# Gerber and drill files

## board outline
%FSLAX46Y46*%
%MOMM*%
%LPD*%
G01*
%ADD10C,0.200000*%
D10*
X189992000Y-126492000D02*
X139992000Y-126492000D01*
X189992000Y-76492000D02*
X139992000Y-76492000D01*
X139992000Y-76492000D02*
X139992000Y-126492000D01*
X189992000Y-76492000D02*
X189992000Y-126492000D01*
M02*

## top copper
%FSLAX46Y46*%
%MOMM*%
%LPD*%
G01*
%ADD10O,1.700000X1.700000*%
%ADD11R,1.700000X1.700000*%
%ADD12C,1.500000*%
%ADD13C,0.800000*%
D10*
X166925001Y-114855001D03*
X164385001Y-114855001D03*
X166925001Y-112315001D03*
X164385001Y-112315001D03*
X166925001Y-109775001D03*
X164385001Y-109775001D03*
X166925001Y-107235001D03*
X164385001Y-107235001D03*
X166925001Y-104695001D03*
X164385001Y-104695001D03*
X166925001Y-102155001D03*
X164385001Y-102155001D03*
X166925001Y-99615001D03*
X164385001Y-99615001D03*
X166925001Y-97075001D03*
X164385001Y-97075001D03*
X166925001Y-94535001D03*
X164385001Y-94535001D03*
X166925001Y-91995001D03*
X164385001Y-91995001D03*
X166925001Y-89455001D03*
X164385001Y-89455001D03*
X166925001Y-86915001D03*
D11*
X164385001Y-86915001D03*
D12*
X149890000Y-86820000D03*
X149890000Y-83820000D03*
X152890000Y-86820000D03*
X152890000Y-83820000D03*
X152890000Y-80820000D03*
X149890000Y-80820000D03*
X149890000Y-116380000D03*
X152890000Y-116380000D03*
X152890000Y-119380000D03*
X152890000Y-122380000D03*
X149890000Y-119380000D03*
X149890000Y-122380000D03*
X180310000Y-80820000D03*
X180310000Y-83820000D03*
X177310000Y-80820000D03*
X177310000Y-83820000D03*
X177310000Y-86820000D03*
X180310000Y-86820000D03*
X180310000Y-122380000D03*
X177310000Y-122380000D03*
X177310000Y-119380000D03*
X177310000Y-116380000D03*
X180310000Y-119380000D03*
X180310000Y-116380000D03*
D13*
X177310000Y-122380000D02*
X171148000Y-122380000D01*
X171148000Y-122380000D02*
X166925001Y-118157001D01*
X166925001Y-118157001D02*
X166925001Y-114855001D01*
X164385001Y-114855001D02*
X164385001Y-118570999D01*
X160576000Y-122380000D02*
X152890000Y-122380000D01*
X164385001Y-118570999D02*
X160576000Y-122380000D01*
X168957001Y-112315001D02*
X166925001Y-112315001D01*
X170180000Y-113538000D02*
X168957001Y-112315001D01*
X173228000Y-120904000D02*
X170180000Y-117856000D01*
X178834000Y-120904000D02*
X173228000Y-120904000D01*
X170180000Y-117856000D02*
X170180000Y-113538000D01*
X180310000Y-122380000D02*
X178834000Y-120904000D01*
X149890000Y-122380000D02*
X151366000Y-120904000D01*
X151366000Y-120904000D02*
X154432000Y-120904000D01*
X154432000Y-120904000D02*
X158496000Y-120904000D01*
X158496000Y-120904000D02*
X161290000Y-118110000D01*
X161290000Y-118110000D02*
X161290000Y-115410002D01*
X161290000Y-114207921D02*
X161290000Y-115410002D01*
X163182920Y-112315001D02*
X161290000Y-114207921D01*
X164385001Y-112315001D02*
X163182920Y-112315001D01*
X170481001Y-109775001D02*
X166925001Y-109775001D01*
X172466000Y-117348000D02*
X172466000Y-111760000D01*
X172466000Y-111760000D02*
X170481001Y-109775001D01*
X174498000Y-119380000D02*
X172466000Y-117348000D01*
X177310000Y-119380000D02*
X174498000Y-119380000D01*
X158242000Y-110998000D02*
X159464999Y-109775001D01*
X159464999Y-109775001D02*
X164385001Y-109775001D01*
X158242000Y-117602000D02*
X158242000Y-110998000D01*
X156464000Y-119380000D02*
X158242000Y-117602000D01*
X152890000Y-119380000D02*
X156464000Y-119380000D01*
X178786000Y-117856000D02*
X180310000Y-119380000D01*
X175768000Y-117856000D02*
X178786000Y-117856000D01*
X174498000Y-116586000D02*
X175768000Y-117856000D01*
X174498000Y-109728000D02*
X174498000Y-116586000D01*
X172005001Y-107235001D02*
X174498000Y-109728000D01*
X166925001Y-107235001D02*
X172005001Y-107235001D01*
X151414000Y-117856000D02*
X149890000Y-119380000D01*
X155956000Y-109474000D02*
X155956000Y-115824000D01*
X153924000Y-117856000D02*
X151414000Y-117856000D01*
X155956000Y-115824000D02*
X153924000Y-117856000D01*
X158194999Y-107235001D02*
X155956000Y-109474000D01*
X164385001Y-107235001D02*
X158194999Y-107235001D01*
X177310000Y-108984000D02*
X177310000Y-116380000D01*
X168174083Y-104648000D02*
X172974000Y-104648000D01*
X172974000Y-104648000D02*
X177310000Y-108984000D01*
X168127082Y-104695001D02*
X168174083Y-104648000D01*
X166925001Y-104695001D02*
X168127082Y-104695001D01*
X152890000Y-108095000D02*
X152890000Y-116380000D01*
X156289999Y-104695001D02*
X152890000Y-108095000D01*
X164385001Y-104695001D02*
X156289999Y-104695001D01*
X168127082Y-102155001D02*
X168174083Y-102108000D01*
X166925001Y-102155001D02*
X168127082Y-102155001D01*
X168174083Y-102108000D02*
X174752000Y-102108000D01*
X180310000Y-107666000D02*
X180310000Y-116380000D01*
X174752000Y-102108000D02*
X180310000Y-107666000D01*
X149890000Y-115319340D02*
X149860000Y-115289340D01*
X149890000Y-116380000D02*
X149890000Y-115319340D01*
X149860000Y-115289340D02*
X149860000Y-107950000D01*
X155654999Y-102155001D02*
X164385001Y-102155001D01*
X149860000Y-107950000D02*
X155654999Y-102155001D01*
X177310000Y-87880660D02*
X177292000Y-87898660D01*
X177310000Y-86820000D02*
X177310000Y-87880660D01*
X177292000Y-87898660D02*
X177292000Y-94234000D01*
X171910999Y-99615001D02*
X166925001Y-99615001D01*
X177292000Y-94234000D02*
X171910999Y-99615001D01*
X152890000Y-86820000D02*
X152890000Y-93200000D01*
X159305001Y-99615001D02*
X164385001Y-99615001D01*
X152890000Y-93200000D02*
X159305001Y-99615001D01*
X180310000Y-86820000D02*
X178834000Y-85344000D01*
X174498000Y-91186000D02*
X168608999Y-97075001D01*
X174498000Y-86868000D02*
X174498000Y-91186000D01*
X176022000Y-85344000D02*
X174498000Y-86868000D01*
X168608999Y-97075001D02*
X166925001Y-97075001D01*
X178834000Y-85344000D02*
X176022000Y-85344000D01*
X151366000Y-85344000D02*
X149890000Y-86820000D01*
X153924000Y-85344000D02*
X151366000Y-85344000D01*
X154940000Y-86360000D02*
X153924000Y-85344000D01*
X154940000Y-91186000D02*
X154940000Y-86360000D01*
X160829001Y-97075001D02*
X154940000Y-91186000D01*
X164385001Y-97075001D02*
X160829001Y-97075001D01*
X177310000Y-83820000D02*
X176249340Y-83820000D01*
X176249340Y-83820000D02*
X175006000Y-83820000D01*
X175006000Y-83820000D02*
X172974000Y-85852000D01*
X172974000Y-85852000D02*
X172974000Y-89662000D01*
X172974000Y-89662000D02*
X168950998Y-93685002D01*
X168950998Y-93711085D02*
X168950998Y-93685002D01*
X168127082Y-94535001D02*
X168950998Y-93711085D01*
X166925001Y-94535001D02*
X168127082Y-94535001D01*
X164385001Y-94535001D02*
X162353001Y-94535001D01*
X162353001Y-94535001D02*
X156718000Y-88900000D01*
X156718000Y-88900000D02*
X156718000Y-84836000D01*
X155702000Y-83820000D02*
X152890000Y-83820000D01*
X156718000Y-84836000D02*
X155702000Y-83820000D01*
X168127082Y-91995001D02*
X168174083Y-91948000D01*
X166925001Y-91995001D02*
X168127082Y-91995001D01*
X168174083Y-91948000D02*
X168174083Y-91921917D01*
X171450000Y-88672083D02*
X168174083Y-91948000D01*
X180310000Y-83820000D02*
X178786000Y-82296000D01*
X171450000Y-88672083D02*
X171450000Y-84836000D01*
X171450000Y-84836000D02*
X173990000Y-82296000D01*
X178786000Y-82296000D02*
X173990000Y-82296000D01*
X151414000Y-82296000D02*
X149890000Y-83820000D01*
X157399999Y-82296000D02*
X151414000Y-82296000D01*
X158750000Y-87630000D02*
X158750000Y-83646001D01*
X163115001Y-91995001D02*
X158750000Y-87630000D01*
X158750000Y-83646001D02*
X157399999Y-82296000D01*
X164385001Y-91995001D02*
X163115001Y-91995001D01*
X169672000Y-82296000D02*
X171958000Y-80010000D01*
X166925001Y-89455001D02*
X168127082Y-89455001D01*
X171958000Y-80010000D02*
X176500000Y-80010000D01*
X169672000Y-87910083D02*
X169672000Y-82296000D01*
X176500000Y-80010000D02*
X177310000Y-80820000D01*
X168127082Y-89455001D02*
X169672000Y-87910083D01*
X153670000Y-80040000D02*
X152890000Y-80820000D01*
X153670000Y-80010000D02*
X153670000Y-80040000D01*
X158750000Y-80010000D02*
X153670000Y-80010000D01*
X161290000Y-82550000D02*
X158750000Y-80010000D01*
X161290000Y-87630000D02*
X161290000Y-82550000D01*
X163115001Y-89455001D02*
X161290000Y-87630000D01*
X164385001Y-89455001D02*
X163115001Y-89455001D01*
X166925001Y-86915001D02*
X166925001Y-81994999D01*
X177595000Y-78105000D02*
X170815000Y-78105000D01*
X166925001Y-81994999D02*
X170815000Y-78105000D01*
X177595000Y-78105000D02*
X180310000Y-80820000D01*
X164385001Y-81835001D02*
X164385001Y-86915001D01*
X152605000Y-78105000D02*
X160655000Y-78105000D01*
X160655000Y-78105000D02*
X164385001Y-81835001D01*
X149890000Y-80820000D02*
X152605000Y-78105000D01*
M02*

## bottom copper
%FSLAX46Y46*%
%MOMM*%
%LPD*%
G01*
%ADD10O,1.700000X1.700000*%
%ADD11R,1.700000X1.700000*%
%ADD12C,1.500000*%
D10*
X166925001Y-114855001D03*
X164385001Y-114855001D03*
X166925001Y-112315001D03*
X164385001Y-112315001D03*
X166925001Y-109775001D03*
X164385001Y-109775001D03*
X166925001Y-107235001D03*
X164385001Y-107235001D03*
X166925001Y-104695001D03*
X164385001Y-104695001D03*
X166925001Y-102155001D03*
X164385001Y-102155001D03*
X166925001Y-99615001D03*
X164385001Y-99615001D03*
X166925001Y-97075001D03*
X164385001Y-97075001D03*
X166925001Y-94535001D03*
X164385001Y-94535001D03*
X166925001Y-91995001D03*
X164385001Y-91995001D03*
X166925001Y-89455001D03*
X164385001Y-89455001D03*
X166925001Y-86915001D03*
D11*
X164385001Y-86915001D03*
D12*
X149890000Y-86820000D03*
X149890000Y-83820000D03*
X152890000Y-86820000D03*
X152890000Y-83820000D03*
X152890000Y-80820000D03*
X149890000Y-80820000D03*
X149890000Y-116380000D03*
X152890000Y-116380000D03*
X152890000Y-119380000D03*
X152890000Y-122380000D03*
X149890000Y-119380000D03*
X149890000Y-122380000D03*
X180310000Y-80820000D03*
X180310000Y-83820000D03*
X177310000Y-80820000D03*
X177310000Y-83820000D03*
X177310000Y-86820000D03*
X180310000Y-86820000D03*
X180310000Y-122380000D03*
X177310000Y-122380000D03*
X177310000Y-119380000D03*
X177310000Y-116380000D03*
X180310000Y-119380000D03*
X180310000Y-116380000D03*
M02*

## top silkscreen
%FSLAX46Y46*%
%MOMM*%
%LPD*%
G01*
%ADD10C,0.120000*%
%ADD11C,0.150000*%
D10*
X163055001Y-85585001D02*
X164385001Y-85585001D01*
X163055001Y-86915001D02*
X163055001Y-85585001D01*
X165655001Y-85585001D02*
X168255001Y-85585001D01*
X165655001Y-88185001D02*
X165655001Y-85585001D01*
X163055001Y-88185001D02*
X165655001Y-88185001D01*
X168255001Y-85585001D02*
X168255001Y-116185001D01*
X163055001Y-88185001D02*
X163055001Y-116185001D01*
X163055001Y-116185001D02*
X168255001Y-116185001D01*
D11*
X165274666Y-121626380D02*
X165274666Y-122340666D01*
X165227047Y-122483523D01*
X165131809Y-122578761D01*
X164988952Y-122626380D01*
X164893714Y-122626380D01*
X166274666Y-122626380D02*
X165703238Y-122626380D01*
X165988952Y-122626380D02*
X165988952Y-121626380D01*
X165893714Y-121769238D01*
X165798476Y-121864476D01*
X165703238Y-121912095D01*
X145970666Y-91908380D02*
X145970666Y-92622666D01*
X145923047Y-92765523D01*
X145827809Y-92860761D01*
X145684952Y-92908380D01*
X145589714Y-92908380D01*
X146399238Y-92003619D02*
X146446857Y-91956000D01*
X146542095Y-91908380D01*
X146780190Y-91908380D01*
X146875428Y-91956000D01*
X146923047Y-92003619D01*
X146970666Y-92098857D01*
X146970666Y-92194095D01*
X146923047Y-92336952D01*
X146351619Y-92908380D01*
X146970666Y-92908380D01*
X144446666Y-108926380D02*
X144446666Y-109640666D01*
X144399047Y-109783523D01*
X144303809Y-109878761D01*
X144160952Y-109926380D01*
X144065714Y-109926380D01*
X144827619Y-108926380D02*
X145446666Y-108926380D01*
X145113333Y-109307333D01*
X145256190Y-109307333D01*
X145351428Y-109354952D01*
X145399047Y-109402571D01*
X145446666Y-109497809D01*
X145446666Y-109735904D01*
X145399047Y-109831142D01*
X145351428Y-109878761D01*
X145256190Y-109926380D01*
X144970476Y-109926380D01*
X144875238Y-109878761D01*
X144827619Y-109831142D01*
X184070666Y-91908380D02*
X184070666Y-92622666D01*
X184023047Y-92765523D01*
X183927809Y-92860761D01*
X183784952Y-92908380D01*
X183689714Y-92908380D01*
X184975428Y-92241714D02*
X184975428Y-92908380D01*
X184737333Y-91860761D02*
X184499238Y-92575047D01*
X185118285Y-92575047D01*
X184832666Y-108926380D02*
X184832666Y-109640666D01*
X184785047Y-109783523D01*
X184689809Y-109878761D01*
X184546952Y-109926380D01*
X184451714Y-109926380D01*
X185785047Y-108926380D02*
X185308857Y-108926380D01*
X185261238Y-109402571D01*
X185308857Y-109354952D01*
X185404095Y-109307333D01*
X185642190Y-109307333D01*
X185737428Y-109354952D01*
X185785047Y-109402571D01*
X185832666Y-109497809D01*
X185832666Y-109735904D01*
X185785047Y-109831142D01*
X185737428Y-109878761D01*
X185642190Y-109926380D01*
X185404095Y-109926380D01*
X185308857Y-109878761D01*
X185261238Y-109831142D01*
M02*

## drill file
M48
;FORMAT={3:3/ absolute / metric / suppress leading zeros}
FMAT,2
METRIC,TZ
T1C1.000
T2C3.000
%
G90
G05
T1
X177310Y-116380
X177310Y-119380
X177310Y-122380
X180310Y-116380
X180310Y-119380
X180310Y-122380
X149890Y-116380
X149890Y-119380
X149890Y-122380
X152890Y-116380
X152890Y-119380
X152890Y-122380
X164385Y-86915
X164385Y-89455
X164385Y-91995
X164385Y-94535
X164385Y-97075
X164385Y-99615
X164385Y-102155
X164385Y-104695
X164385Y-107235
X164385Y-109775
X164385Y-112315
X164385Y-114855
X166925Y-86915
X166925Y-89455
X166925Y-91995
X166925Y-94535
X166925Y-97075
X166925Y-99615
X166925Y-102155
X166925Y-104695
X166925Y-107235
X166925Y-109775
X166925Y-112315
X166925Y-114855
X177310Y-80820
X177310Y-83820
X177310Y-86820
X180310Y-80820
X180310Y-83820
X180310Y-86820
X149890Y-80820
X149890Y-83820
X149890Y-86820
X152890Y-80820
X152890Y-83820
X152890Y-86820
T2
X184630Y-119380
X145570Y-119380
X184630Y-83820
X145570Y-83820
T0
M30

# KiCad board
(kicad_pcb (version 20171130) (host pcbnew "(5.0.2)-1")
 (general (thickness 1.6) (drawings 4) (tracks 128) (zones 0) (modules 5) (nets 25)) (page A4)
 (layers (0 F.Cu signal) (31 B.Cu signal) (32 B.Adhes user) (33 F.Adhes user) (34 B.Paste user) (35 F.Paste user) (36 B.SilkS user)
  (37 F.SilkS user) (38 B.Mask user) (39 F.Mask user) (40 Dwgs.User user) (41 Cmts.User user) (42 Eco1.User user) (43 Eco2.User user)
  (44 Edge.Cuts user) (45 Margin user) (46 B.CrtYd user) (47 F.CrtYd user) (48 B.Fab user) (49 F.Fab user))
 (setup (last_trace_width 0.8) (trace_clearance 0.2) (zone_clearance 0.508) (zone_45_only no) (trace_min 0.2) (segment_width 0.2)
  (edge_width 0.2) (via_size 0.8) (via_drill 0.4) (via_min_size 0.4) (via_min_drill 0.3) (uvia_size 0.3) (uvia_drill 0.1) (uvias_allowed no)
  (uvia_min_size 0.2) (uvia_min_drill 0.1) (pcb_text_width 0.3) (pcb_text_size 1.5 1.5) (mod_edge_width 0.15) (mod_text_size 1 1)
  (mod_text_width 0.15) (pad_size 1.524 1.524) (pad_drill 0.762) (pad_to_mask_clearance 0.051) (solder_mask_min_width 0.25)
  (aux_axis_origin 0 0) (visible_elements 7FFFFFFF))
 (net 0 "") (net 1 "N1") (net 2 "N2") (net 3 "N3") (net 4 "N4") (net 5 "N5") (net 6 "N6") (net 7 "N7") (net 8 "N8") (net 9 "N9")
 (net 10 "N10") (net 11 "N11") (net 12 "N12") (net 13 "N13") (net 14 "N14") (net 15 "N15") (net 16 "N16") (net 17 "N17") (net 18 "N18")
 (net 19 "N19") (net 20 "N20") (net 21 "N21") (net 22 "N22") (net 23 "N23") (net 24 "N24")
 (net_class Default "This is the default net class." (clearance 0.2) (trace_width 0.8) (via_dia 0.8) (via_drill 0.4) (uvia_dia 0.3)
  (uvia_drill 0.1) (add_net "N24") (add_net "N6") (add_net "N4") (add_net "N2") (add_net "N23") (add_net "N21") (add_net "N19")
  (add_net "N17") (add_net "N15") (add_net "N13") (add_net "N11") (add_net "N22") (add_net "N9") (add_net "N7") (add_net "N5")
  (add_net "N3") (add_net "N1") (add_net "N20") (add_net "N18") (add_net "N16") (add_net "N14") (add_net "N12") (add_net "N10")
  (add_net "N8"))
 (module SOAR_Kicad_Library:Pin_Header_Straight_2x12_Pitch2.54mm (layer F.Cu) (at 164.385001 86.915001)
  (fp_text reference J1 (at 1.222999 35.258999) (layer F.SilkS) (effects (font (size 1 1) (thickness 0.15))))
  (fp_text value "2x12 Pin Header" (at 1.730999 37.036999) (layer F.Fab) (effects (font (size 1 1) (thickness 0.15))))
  (fp_line (start -1.33 -1.33) (end 0 -1.33) (layer F.SilkS) (width 0.12))
  (fp_line (start -1.33 0) (end -1.33 -1.33) (layer F.SilkS) (width 0.12))
  (fp_line (start 1.27 -1.33) (end 3.87 -1.33) (layer F.SilkS) (width 0.12))
  (fp_line (start 1.27 1.27) (end 1.27 -1.33) (layer F.SilkS) (width 0.12))
  (fp_line (start -1.33 1.27) (end 1.27 1.27) (layer F.SilkS) (width 0.12))
  (fp_line (start 3.87 -1.33) (end 3.87 29.27) (layer F.SilkS) (width 0.12))
  (fp_line (start -1.33 1.27) (end -1.33 29.27) (layer F.SilkS) (width 0.12))
  (fp_line (start -1.33 29.27) (end 3.87 29.27) (layer F.SilkS) (width 0.12))
  (pad 24 thru_hole oval (at 2.54 27.94) (size 1.7 1.7) (drill 1) (layers *.Cu *.Mask) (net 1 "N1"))
  (pad 12 thru_hole oval (at 0 27.94) (size 1.7 1.7) (drill 1) (layers *.Cu *.Mask) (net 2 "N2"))
  (pad 23 thru_hole oval (at 2.54 25.4) (size 1.7 1.7) (drill 1) (layers *.Cu *.Mask) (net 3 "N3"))
  (pad 11 thru_hole oval (at 0 25.4) (size 1.7 1.7) (drill 1) (layers *.Cu *.Mask) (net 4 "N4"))
  (pad 22 thru_hole oval (at 2.54 22.86) (size 1.7 1.7) (drill 1) (layers *.Cu *.Mask) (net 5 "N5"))
  (pad 10 thru_hole oval (at 0 22.86) (size 1.7 1.7) (drill 1) (layers *.Cu *.Mask) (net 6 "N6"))
  (pad 21 thru_hole oval (at 2.54 20.32) (size 1.7 1.7) (drill 1) (layers *.Cu *.Mask) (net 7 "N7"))
  (pad 9 thru_hole oval (at 0 20.32) (size 1.7 1.7) (drill 1) (layers *.Cu *.Mask) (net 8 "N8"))
  (pad 20 thru_hole oval (at 2.54 17.78) (size 1.7 1.7) (drill 1) (layers *.Cu *.Mask) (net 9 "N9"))
  (pad 8 thru_hole oval (at 0 17.78) (size 1.7 1.7) (drill 1) (layers *.Cu *.Mask) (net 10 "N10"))
  (pad 19 thru_hole oval (at 2.54 15.24) (size 1.7 1.7) (drill 1) (layers *.Cu *.Mask) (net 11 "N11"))
  (pad 7 thru_hole oval (at 0 15.24) (size 1.7 1.7) (drill 1) (layers *.Cu *.Mask) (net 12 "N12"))
  (pad 18 thru_hole oval (at 2.54 12.7) (size 1.7 1.7) (drill 1) (layers *.Cu *.Mask) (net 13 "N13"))
  (pad 6 thru_hole oval (at 0 12.7) (size 1.7 1.7) (drill 1) (layers *.Cu *.Mask) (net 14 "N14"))
  (pad 17 thru_hole oval (at 2.54 10.16) (size 1.7 1.7) (drill 1) (layers *.Cu *.Mask) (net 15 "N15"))
  (pad 5 thru_hole oval (at 0 10.16) (size 1.7 1.7) (drill 1) (layers *.Cu *.Mask) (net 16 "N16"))
  (pad 16 thru_hole oval (at 2.54 7.62) (size 1.7 1.7) (drill 1) (layers *.Cu *.Mask) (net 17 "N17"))
  (pad 4 thru_hole oval (at 0 7.62) (size 1.7 1.7) (drill 1) (layers *.Cu *.Mask) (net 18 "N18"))
  (pad 15 thru_hole oval (at 2.54 5.08) (size 1.7 1.7) (drill 1) (layers *.Cu *.Mask) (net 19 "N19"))
  (pad 3 thru_hole oval (at 0 5.08) (size 1.7 1.7) (drill 1) (layers *.Cu *.Mask) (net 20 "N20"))
  (pad 14 thru_hole oval (at 2.54 2.54) (size 1.7 1.7) (drill 1) (layers *.Cu *.Mask) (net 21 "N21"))
  (pad 2 thru_hole oval (at 0 2.54) (size 1.7 1.7) (drill 1) (layers *.Cu *.Mask) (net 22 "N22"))
  (pad 13 thru_hole oval (at 2.54 0) (size 1.7 1.7) (drill 1) (layers *.Cu *.Mask) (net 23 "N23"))
  (pad 1 thru_hole rect (at 0 0) (size 1.7 1.7) (drill 1) (layers *.Cu *.Mask) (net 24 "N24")))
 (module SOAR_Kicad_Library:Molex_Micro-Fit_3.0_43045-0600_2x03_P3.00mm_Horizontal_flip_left (layer F.Cu) (at 140.97 83.82 270)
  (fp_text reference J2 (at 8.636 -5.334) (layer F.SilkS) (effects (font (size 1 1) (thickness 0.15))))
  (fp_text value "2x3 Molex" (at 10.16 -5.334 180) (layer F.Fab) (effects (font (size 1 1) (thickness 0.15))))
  (pad "" np_thru_hole circle (at 0 -4.6 90) (size 3 3) (drill 3) (layers *.Cu *.Mask))
  (pad 5 thru_hole circle (at 3 -8.92 90) (size 1.5 1.5) (drill 1) (layers *.Cu *.Mask) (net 16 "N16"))
  (pad 3 thru_hole circle (at 0 -8.92 90) (size 1.5 1.5) (drill 1) (layers *.Cu *.Mask) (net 20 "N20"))
  (pad 6 thru_hole circle (at 3 -11.92 90) (size 1.5 1.5) (drill 1) (layers *.Cu *.Mask) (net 14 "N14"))
  (pad 4 thru_hole circle (at 0 -11.92 90) (size 1.5 1.5) (drill 1) (layers *.Cu *.Mask) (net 18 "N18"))
  (pad 2 thru_hole circle (at -3 -11.92 90) (size 1.5 1.5) (drill 1) (layers *.Cu *.Mask) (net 22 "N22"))
  (pad 1 thru_hole circle (at -3 -8.92 90) (size 1.5 1.5) (drill 1) (layers *.Cu *.Mask) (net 24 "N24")))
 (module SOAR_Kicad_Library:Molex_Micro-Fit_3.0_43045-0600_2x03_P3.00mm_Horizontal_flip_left (layer F.Cu) (at 140.97 119.38 270)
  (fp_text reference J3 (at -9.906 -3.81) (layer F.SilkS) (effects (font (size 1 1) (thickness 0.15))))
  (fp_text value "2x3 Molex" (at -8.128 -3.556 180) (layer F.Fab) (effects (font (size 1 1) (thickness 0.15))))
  (pad 1 thru_hole circle (at -3 -8.92 90) (size 1.5 1.5) (drill 1) (layers *.Cu *.Mask) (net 12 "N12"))
  (pad 2 thru_hole circle (at -3 -11.92 90) (size 1.5 1.5) (drill 1) (layers *.Cu *.Mask) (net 10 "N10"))
  (pad 4 thru_hole circle (at 0 -11.92 90) (size 1.5 1.5) (drill 1) (layers *.Cu *.Mask) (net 6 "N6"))
  (pad 6 thru_hole circle (at 3 -11.92 90) (size 1.5 1.5) (drill 1) (layers *.Cu *.Mask) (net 2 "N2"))
  (pad 3 thru_hole circle (at 0 -8.92 90) (size 1.5 1.5) (drill 1) (layers *.Cu *.Mask) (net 8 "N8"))
  (pad 5 thru_hole circle (at 3 -8.92 90) (size 1.5 1.5) (drill 1) (layers *.Cu *.Mask) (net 4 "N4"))
  (pad "" np_thru_hole circle (at 0 -4.6 90) (size 3 3) (drill 3) (layers *.Cu *.Mask)))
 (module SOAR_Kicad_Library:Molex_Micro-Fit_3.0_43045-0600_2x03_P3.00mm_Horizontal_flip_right (layer F.Cu) (at 189.23 83.82 90)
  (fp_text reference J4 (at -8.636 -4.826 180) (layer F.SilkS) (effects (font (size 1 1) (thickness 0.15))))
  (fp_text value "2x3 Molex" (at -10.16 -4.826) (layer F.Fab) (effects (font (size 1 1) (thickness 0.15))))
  (pad "" np_thru_hole circle (at 0 -4.6 270) (size 3 3) (drill 3) (layers *.Cu *.Mask))
  (pad 1 thru_hole circle (at 3 -8.92 270) (size 1.5 1.5) (drill 1) (layers *.Cu *.Mask) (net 23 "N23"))
  (pad 3 thru_hole circle (at 0 -8.92 270) (size 1.5 1.5) (drill 1) (layers *.Cu *.Mask) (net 19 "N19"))
  (pad 2 thru_hole circle (at 3 -11.92 270) (size 1.5 1.5) (drill 1) (layers *.Cu *.Mask) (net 21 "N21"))
  (pad 4 thru_hole circle (at 0 -11.92 270) (size 1.5 1.5) (drill 1) (layers *.Cu *.Mask) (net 17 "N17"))
  (pad 6 thru_hole circle (at -3 -11.92 270) (size 1.5 1.5) (drill 1) (layers *.Cu *.Mask) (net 13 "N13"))
  (pad 5 thru_hole circle (at -3 -8.92 270) (size 1.5 1.5) (drill 1) (layers *.Cu *.Mask) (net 15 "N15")))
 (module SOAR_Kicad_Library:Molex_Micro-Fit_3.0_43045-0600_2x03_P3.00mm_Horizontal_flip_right (layer F.Cu) (at 189.23 119.38 90)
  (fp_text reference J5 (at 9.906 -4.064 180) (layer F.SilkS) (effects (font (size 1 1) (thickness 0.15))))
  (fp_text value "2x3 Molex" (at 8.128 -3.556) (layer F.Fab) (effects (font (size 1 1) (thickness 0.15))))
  (pad 5 thru_hole circle (at -3 -8.92 270) (size 1.5 1.5) (drill 1) (layers *.Cu *.Mask) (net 3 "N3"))
  (pad 6 thru_hole circle (at -3 -11.92 270) (size 1.5 1.5) (drill 1) (layers *.Cu *.Mask) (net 1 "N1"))
  (pad 4 thru_hole circle (at 0 -11.92 270) (size 1.5 1.5) (drill 1) (layers *.Cu *.Mask) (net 5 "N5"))
  (pad 2 thru_hole circle (at 3 -11.92 270) (size 1.5 1.5) (drill 1) (layers *.Cu *.Mask) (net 9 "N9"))
  (pad 3 thru_hole circle (at 0 -8.92 270) (size 1.5 1.5) (drill 1) (layers *.Cu *.Mask) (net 7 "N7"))
  (pad 1 thru_hole circle (at 3 -8.92 270) (size 1.5 1.5) (drill 1) (layers *.Cu *.Mask) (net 11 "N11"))
  (pad "" np_thru_hole circle (at 0 -4.6 270) (size 3 3) (drill 3) (layers *.Cu *.Mask)))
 (gr_line (start 189.992 126.492) (end 139.992 126.492) (layer Edge.Cuts) (width 0.2))
 (gr_line (start 189.992 76.492) (end 139.992 76.492) (layer Edge.Cuts) (width 0.2))
 (gr_line (start 139.992 76.492) (end 139.992 126.492) (layer Edge.Cuts) (width 0.2))
 (gr_line (start 189.992 76.492) (end 189.992 126.492) (layer Edge.Cuts) (width 0.2))
 (segment (start 177.31 122.38) (end 171.148 122.38) (width 0.8) (layer F.Cu) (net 1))
 (segment (start 171.148 122.38) (end 166.925001 118.157001) (width 0.8) (layer F.Cu) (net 1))
 (segment (start 166.925001 118.157001) (end 166.925001 114.855001) (width 0.8) (layer F.Cu) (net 1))
 (segment (start 164.385001 114.855001) (end 164.385001 118.570999) (width 0.8) (layer F.Cu) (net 2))
 (segment (start 160.576 122.38) (end 152.89 122.38) (width 0.8) (layer F.Cu) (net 2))
 (segment (start 164.385001 118.570999) (end 160.576 122.38) (width 0.8) (layer F.Cu) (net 2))
 (segment (start 168.957001 112.315001) (end 166.925001 112.315001) (width 0.8) (layer F.Cu) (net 3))
 (segment (start 170.18 113.538) (end 168.957001 112.315001) (width 0.8) (layer F.Cu) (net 3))
 (segment (start 173.228 120.904) (end 170.18 117.856) (width 0.8) (layer F.Cu) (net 3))
 (segment (start 178.834 120.904) (end 173.228 120.904) (width 0.8) (layer F.Cu) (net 3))
 (segment (start 170.18 117.856) (end 170.18 113.538) (width 0.8) (layer F.Cu) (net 3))
 (segment (start 180.31 122.38) (end 178.834 120.904) (width 0.8) (layer F.Cu) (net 3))
 (segment (start 149.89 122.38) (end 151.366 120.904) (width 0.8) (layer F.Cu) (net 4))
 (segment (start 151.366 120.904) (end 154.432 120.904) (width 0.8) (layer F.Cu) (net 4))
 (segment (start 154.432 120.904) (end 158.496 120.904) (width 0.8) (layer F.Cu) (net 4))
 (segment (start 158.496 120.904) (end 161.29 118.11) (width 0.8) (layer F.Cu) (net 4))
 (segment (start 161.29 118.11) (end 161.29 115.410002) (width 0.8) (layer F.Cu) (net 4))
 (segment (start 161.29 114.207921) (end 161.29 115.410002) (width 0.8) (layer F.Cu) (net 4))
 (segment (start 163.18292 112.315001) (end 161.29 114.207921) (width 0.8) (layer F.Cu) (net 4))
 (segment (start 164.385001 112.315001) (end 163.18292 112.315001) (width 0.8) (layer F.Cu) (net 4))
 (segment (start 170.481001 109.775001) (end 166.925001 109.775001) (width 0.8) (layer F.Cu) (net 5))
 (segment (start 172.466 117.348) (end 172.466 111.76) (width 0.8) (layer F.Cu) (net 5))
 (segment (start 172.466 111.76) (end 170.481001 109.775001) (width 0.8) (layer F.Cu) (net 5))
 (segment (start 174.498 119.38) (end 172.466 117.348) (width 0.8) (layer F.Cu) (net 5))
 (segment (start 177.31 119.38) (end 174.498 119.38) (width 0.8) (layer F.Cu) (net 5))
 (segment (start 158.242 110.998) (end 159.464999 109.775001) (width 0.8) (layer F.Cu) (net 6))
 (segment (start 159.464999 109.775001) (end 164.385001 109.775001) (width 0.8) (layer F.Cu) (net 6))
 (segment (start 158.242 117.602) (end 158.242 110.998) (width 0.8) (layer F.Cu) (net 6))
 (segment (start 156.464 119.38) (end 158.242 117.602) (width 0.8) (layer F.Cu) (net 6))
 (segment (start 152.89 119.38) (end 156.464 119.38) (width 0.8) (layer F.Cu) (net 6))
 (segment (start 178.786 117.856) (end 180.31 119.38) (width 0.8) (layer F.Cu) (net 7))
 (segment (start 175.768 117.856) (end 178.786 117.856) (width 0.8) (layer F.Cu) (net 7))
 (segment (start 174.498 116.586) (end 175.768 117.856) (width 0.8) (layer F.Cu) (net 7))
 (segment (start 174.498 109.728) (end 174.498 116.586) (width 0.8) (layer F.Cu) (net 7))
 (segment (start 172.005001 107.235001) (end 174.498 109.728) (width 0.8) (layer F.Cu) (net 7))
 (segment (start 166.925001 107.235001) (end 172.005001 107.235001) (width 0.8) (layer F.Cu) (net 7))
 (segment (start 151.414 117.856) (end 149.89 119.38) (width 0.8) (layer F.Cu) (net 8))
 (segment (start 155.956 109.474) (end 155.956 115.824) (width 0.8) (layer F.Cu) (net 8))
 (segment (start 153.924 117.856) (end 151.414 117.856) (width 0.8) (layer F.Cu) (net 8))
 (segment (start 155.956 115.824) (end 153.924 117.856) (width 0.8) (layer F.Cu) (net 8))
 (segment (start 158.194999 107.235001) (end 155.956 109.474) (width 0.8) (layer F.Cu) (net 8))
 (segment (start 164.385001 107.235001) (end 158.194999 107.235001) (width 0.8) (layer F.Cu) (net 8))
 (segment (start 177.31 108.984) (end 177.31 116.38) (width 0.8) (layer F.Cu) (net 9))
 (segment (start 168.174083 104.648) (end 172.974 104.648) (width 0.8) (layer F.Cu) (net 9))
 (segment (start 172.974 104.648) (end 177.31 108.984) (width 0.8) (layer F.Cu) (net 9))
 (segment (start 168.127082 104.695001) (end 168.174083 104.648) (width 0.8) (layer F.Cu) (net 9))
 (segment (start 166.925001 104.695001) (end 168.127082 104.695001) (width 0.8) (layer F.Cu) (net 9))
 (segment (start 152.89 108.095) (end 152.89 116.38) (width 0.8) (layer F.Cu) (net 10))
 (segment (start 156.289999 104.695001) (end 152.89 108.095) (width 0.8) (layer F.Cu) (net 10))
 (segment (start 164.385001 104.695001) (end 156.289999 104.695001) (width 0.8) (layer F.Cu) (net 10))
 (segment (start 168.127082 102.155001) (end 168.174083 102.108) (width 0.8) (layer F.Cu) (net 11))
 (segment (start 166.925001 102.155001) (end 168.127082 102.155001) (width 0.8) (layer F.Cu) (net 11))
 (segment (start 168.174083 102.108) (end 174.752 102.108) (width 0.8) (layer F.Cu) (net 11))
 (segment (start 180.31 107.666) (end 180.31 116.38) (width 0.8) (layer F.Cu) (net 11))
 (segment (start 174.752 102.108) (end 180.31 107.666) (width 0.8) (layer F.Cu) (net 11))
 (segment (start 149.89 115.31934) (end 149.86 115.28934) (width 0.8) (layer F.Cu) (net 12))
 (segment (start 149.89 116.38) (end 149.89 115.31934) (width 0.8) (layer F.Cu) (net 12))
 (segment (start 149.86 115.28934) (end 149.86 107.95) (width 0.8) (layer F.Cu) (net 12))
 (segment (start 155.654999 102.155001) (end 164.385001 102.155001) (width 0.8) (layer F.Cu) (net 12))
 (segment (start 149.86 107.95) (end 155.654999 102.155001) (width 0.8) (layer F.Cu) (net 12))
 (segment (start 177.31 87.88066) (end 177.292 87.89866) (width 0.8) (layer F.Cu) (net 13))
 (segment (start 177.31 86.82) (end 177.31 87.88066) (width 0.8) (layer F.Cu) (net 13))
 (segment (start 177.292 87.89866) (end 177.292 94.234) (width 0.8) (layer F.Cu) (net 13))
 (segment (start 171.910999 99.615001) (end 166.925001 99.615001) (width 0.8) (layer F.Cu) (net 13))
 (segment (start 177.292 94.234) (end 171.910999 99.615001) (width 0.8) (layer F.Cu) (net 13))
 (segment (start 152.89 86.82) (end 152.89 93.2) (width 0.8) (layer F.Cu) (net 14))
 (segment (start 159.305001 99.615001) (end 164.385001 99.615001) (width 0.8) (layer F.Cu) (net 14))
 (segment (start 152.89 93.2) (end 159.305001 99.615001) (width 0.8) (layer F.Cu) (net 14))
 (segment (start 180.31 86.82) (end 178.834 85.344) (width 0.8) (layer F.Cu) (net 15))
 (segment (start 174.498 91.186) (end 168.608999 97.075001) (width 0.8) (layer F.Cu) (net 15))
 (segment (start 174.498 86.868) (end 174.498 91.186) (width 0.8) (layer F.Cu) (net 15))
 (segment (start 176.022 85.344) (end 174.498 86.868) (width 0.8) (layer F.Cu) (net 15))
 (segment (start 168.608999 97.075001) (end 166.925001 97.075001) (width 0.8) (layer F.Cu) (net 15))
 (segment (start 178.834 85.344) (end 176.022 85.344) (width 0.8) (layer F.Cu) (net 15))
 (segment (start 151.366 85.344) (end 149.89 86.82) (width 0.8) (layer F.Cu) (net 16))
 (segment (start 153.924 85.344) (end 151.366 85.344) (width 0.8) (layer F.Cu) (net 16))
 (segment (start 154.94 86.36) (end 153.924 85.344) (width 0.8) (layer F.Cu) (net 16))
 (segment (start 154.94 91.186) (end 154.94 86.36) (width 0.8) (layer F.Cu) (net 16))
 (segment (start 160.829001 97.075001) (end 154.94 91.186) (width 0.8) (layer F.Cu) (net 16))
 (segment (start 164.385001 97.075001) (end 160.829001 97.075001) (width 0.8) (layer F.Cu) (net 16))
 (segment (start 177.31 83.82) (end 176.24934 83.82) (width 0.8) (layer F.Cu) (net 17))
 (segment (start 176.24934 83.82) (end 175.006 83.82) (width 0.8) (layer F.Cu) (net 17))
 (segment (start 175.006 83.82) (end 172.974 85.852) (width 0.8) (layer F.Cu) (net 17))
 (segment (start 172.974 85.852) (end 172.974 89.662) (width 0.8) (layer F.Cu) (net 17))
 (segment (start 172.974 89.662) (end 168.950998 93.685002) (width 0.8) (layer F.Cu) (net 17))
 (segment (start 168.950998 93.711085) (end 168.950998 93.685002) (width 0.8) (layer F.Cu) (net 17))
 (segment (start 168.127082 94.535001) (end 168.950998 93.711085) (width 0.8) (layer F.Cu) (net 17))
 (segment (start 166.925001 94.535001) (end 168.127082 94.535001) (width 0.8) (layer F.Cu) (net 17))
 (segment (start 164.385001 94.535001) (end 162.353001 94.535001) (width 0.8) (layer F.Cu) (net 18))
 (segment (start 162.353001 94.535001) (end 156.718 88.9) (width 0.8) (layer F.Cu) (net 18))
 (segment (start 156.718 88.9) (end 156.718 84.836) (width 0.8) (layer F.Cu) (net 18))
 (segment (start 155.702 83.82) (end 152.89 83.82) (width 0.8) (layer F.Cu) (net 18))
 (segment (start 156.718 84.836) (end 155.702 83.82) (width 0.8) (layer F.Cu) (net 18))
 (segment (start 168.127082 91.995001) (end 168.174083 91.948) (width 0.8) (layer F.Cu) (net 19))
 (segment (start 166.925001 91.995001) (end 168.127082 91.995001) (width 0.8) (layer F.Cu) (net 19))
 (segment (start 168.174083 91.948) (end 168.174083 91.921917) (width 0.8) (layer F.Cu) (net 19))
 (segment (start 171.45 88.672083) (end 168.174083 91.948) (width 0.8) (layer F.Cu) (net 19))
 (segment (start 180.31 83.82) (end 178.786 82.296) (width 0.8) (layer F.Cu) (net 19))
 (segment (start 171.45 88.672083) (end 171.45 84.836) (width 0.8) (layer F.Cu) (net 19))
 (segment (start 171.45 84.836) (end 173.99 82.296) (width 0.8) (layer F.Cu) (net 19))
 (segment (start 178.786 82.296) (end 173.99 82.296) (width 0.8) (layer F.Cu) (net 19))
 (segment (start 151.414 82.296) (end 149.89 83.82) (width 0.8) (layer F.Cu) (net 20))
 (segment (start 157.399999 82.296) (end 151.414 82.296) (width 0.8) (layer F.Cu) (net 20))
 (segment (start 158.75 87.63) (end 158.75 83.646001) (width 0.8) (layer F.Cu) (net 20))
 (segment (start 163.115001 91.995001) (end 158.75 87.63) (width 0.8) (layer F.Cu) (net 20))
 (segment (start 158.75 83.646001) (end 157.399999 82.296) (width 0.8) (layer F.Cu) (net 20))
 (segment (start 164.385001 91.995001) (end 163.115001 91.995001) (width 0.8) (layer F.Cu) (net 20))
 (segment (start 169.672 82.296) (end 171.958 80.01) (width 0.8) (layer F.Cu) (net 21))
 (segment (start 166.925001 89.455001) (end 168.127082 89.455001) (width 0.8) (layer F.Cu) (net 21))
 (segment (start 171.958 80.01) (end 176.5 80.01) (width 0.8) (layer F.Cu) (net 21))
 (segment (start 169.672 87.910083) (end 169.672 82.296) (width 0.8) (layer F.Cu) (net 21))
 (segment (start 176.5 80.01) (end 177.31 80.82) (width 0.8) (layer F.Cu) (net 21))
 (segment (start 168.127082 89.455001) (end 169.672 87.910083) (width 0.8) (layer F.Cu) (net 21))
 (segment (start 153.67 80.04) (end 152.89 80.82) (width 0.8) (layer F.Cu) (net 22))
 (segment (start 153.67 80.01) (end 153.67 80.04) (width 0.8) (layer F.Cu) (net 22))
 (segment (start 158.75 80.01) (end 153.67 80.01) (width 0.8) (layer F.Cu) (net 22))
 (segment (start 161.29 82.55) (end 158.75 80.01) (width 0.8) (layer F.Cu) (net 22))
 (segment (start 161.29 87.63) (end 161.29 82.55) (width 0.8) (layer F.Cu) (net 22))
 (segment (start 163.115001 89.455001) (end 161.29 87.63) (width 0.8) (layer F.Cu) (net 22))
 (segment (start 164.385001 89.455001) (end 163.115001 89.455001) (width 0.8) (layer F.Cu) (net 22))
 (segment (start 166.925001 86.915001) (end 166.925001 81.994999) (width 0.8) (layer F.Cu) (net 23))
 (segment (start 177.595 78.105) (end 170.815 78.105) (width 0.8) (layer F.Cu) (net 23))
 (segment (start 166.925001 81.994999) (end 170.815 78.105) (width 0.8) (layer F.Cu) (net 23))
 (segment (start 177.595 78.105) (end 180.31 80.82) (width 0.8) (layer F.Cu) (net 23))
 (segment (start 164.385001 81.835001) (end 164.385001 86.915001) (width 0.8) (layer F.Cu) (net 24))
 (segment (start 152.605 78.105) (end 160.655 78.105) (width 0.8) (layer F.Cu) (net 24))
 (segment (start 160.655 78.105) (end 164.385001 81.835001) (width 0.8) (layer F.Cu) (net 24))
 (segment (start 149.89 80.82) (end 152.605 78.105) (width 0.8) (layer F.Cu) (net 24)))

